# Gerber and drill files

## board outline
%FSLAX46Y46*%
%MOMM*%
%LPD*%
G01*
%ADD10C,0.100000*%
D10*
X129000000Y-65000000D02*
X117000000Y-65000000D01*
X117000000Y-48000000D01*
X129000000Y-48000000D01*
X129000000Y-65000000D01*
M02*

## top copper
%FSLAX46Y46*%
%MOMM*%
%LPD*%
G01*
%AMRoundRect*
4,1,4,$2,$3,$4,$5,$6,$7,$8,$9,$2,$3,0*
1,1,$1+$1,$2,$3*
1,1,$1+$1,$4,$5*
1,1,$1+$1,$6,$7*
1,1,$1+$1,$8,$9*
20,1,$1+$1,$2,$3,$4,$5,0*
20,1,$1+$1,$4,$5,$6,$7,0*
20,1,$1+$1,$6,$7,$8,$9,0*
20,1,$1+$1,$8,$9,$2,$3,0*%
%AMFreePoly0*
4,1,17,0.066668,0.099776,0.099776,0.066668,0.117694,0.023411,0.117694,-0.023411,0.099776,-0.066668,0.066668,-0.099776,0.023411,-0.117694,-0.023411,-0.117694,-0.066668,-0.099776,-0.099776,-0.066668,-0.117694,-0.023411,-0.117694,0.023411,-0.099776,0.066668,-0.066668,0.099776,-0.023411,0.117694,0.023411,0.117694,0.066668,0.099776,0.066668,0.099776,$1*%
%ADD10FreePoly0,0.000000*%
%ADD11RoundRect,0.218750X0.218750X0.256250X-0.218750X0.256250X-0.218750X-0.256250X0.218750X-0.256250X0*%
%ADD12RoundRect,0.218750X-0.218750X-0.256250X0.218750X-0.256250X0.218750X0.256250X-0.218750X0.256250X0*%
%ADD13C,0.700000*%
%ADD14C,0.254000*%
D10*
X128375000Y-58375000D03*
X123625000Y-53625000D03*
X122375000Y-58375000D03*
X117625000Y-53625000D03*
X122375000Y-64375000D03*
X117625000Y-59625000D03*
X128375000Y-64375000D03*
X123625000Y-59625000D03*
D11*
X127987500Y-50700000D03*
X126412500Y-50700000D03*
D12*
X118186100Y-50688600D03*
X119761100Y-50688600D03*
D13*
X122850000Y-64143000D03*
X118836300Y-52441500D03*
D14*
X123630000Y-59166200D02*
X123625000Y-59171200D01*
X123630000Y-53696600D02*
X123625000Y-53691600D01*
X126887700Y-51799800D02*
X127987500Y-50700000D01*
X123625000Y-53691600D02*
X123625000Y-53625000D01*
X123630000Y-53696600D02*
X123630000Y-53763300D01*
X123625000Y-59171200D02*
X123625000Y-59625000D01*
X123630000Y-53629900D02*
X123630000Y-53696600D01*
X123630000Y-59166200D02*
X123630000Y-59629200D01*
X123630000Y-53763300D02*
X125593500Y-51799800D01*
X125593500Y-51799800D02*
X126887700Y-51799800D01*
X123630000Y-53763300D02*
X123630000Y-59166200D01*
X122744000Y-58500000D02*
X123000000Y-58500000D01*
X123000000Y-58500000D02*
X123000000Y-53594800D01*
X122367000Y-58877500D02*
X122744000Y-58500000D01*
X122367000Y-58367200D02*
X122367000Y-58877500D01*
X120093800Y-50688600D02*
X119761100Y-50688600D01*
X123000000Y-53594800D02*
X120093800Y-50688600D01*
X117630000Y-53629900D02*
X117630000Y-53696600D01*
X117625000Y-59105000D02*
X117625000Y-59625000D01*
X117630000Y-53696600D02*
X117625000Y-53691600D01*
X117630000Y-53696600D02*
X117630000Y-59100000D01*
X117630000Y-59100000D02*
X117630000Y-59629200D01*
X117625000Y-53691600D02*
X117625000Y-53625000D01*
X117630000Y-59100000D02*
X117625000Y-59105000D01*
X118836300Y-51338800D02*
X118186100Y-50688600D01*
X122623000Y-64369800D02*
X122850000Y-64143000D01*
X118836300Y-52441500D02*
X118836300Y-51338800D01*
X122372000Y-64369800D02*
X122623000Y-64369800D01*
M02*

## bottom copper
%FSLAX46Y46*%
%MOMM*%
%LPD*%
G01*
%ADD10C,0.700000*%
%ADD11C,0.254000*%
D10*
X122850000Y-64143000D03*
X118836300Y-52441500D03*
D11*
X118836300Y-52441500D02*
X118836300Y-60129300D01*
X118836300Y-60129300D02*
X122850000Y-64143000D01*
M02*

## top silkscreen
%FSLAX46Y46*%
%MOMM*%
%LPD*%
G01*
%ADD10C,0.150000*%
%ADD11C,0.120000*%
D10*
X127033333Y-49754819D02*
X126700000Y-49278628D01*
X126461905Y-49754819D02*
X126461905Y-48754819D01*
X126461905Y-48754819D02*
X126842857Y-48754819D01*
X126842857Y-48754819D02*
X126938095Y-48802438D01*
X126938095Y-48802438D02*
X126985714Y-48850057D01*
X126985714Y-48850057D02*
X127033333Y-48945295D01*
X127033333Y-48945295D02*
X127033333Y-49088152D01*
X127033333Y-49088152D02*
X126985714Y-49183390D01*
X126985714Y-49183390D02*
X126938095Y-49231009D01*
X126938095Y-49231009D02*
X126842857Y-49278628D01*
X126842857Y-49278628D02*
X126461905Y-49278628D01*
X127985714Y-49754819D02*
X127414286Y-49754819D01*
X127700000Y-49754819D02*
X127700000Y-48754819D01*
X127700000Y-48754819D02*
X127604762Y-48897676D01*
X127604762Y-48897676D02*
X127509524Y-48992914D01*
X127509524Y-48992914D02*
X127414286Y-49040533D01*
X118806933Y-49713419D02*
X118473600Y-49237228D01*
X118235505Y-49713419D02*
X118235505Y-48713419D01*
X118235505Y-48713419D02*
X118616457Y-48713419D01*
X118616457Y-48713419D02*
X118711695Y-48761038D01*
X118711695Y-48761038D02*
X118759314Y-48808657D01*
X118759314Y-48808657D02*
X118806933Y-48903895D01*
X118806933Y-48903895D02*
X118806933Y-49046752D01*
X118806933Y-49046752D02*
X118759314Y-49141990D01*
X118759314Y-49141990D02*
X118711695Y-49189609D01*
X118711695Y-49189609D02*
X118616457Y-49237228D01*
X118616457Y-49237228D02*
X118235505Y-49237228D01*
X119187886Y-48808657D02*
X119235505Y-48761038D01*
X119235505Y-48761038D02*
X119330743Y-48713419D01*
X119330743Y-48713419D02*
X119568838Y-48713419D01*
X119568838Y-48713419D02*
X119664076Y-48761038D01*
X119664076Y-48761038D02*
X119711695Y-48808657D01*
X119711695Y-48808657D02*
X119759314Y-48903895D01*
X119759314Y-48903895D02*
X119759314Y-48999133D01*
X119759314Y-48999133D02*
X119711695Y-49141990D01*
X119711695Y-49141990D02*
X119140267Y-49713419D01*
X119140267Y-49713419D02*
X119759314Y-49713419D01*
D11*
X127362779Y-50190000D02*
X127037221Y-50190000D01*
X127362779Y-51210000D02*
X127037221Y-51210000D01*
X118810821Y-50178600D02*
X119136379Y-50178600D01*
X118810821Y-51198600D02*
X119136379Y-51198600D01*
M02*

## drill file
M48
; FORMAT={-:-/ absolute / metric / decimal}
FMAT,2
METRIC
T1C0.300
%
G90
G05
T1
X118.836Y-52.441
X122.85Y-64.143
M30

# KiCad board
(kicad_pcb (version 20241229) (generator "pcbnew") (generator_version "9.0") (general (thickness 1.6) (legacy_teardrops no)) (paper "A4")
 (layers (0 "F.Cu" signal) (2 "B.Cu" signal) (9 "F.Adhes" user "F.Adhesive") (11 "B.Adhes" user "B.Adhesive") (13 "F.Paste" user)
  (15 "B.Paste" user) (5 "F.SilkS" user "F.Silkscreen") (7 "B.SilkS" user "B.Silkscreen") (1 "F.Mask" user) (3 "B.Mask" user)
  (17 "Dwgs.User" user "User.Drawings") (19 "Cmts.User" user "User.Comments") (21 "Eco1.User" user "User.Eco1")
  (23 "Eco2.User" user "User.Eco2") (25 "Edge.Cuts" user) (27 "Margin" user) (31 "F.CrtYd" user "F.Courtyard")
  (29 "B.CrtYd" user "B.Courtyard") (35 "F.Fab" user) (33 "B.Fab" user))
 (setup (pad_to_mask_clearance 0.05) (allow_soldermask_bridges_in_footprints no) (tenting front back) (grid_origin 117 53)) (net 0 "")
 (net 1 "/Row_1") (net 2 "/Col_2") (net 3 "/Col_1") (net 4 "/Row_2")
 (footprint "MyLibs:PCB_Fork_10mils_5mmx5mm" (layer "F.Cu") (at 123.5 53.5)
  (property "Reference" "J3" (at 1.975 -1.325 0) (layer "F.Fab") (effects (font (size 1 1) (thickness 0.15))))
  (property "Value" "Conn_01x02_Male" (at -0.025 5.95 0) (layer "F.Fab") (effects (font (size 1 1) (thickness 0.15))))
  (pad "1" smd custom (at 4.875 4.875) (size 0.24 0.24) (layers "F.Cu" "F.Mask") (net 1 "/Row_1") (zone_connect 0) (thermal_bridge_angle 90)
   (options (clearance outline) (anchor circle)) (primitives))
  (pad "2" smd custom (at 0.125 0.125) (size 0.24 0.24) (layers "F.Cu" "F.Mask") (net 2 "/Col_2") (zone_connect 0) (thermal_bridge_angle 90)
   (options (clearance outline) (anchor circle)) (primitives)))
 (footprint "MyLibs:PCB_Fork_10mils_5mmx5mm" (layer "F.Cu") (at 117.5 53.5)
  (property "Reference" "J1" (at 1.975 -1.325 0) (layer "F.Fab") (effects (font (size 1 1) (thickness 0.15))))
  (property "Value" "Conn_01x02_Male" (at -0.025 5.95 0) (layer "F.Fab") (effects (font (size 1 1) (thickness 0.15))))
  (pad "1" smd custom (at 4.875 4.875) (size 0.24 0.24) (layers "F.Cu" "F.Mask") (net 1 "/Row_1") (zone_connect 0) (thermal_bridge_angle 90)
   (options (clearance outline) (anchor circle)) (primitives))
  (pad "2" smd custom (at 0.125 0.125) (size 0.24 0.24) (layers "F.Cu" "F.Mask") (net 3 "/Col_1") (zone_connect 0) (thermal_bridge_angle 90)
   (options (clearance outline) (anchor circle)) (primitives)))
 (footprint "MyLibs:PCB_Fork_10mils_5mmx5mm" (layer "F.Cu") (at 117.5 59.5)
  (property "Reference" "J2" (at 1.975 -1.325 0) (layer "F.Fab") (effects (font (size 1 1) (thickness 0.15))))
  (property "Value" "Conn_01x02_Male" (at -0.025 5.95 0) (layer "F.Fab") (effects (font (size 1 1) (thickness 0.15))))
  (pad "1" smd custom (at 4.875 4.875) (size 0.24 0.24) (layers "F.Cu" "F.Mask") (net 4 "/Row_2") (zone_connect 0) (thermal_bridge_angle 90)
   (options (clearance outline) (anchor circle)) (primitives))
  (pad "2" smd custom (at 0.125 0.125) (size 0.24 0.24) (layers "F.Cu" "F.Mask") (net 3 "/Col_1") (zone_connect 0) (thermal_bridge_angle 90)
   (options (clearance outline) (anchor circle)) (primitives)))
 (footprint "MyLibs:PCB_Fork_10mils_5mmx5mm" (layer "F.Cu") (at 123.5 59.5)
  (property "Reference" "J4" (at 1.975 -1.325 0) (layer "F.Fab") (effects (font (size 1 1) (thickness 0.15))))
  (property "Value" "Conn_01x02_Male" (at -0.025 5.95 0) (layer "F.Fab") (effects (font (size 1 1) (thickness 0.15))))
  (pad "1" smd custom (at 4.875 4.875) (size 0.24 0.24) (layers "F.Cu" "F.Mask") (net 4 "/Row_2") (zone_connect 0) (thermal_bridge_angle 90)
   (options (clearance outline) (anchor circle)) (primitives))
  (pad "2" smd custom (at 0.125 0.125) (size 0.24 0.24) (layers "F.Cu" "F.Mask") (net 2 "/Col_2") (zone_connect 0) (thermal_bridge_angle 90)
   (options (clearance outline) (anchor circle)) (primitives)))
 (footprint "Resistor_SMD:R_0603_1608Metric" (layer "F.Cu") (at 127.2 50.7 180)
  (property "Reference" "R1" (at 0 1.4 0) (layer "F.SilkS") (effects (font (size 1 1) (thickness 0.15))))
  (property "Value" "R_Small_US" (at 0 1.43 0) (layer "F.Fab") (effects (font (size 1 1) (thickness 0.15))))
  (fp_line (start -0.162779 0.51) (end 0.162779 0.51) (stroke (width 0.12) (type solid)) (layer "F.SilkS"))
  (fp_line (start -0.162779 -0.51) (end 0.162779 -0.51) (stroke (width 0.12) (type solid)) (layer "F.SilkS"))
  (pad "1" smd roundrect (at -0.7875 0 180) (size 0.875 0.95) (layers "F.Cu" "F.Mask" "F.Paste") (roundrect_rratio 0.25) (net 2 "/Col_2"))
  (pad "2" smd roundrect (at 0.7875 0 180) (size 0.875 0.95) (layers "F.Cu" "F.Mask" "F.Paste") (roundrect_rratio 0.25) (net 3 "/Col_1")))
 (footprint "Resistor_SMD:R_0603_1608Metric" (layer "F.Cu") (at 118.9736 50.6886)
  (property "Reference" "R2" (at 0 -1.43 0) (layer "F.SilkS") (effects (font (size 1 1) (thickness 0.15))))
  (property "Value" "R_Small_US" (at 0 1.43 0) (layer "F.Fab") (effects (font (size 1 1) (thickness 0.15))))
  (fp_line (start -0.162779 -0.51) (end 0.162779 -0.51) (stroke (width 0.12) (type solid)) (layer "F.SilkS"))
  (fp_line (start -0.162779 0.51) (end 0.162779 0.51) (stroke (width 0.12) (type solid)) (layer "F.SilkS"))
  (pad "1" smd roundrect (at -0.7875 0) (size 0.875 0.95) (layers "F.Cu" "F.Mask" "F.Paste") (roundrect_rratio 0.25) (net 4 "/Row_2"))
  (pad "2" smd roundrect (at 0.7875 0) (size 0.875 0.95) (layers "F.Cu" "F.Mask" "F.Paste") (roundrect_rratio 0.25) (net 1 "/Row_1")))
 (gr_poly (pts (xy 129 65) (xy 117 65) (xy 117 48) (xy 129 48)) (stroke (width 0.1) (type solid)) (fill no) (layer "Edge.Cuts"))
 (segment (start 123.63 59.1662) (end 123.625 59.1712) (width 0.254) (layer "F.Cu") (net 2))
 (segment (start 123.63 53.6966) (end 123.625 53.6916) (width 0.254) (layer "F.Cu") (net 2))
 (segment (start 126.8877 51.7998) (end 127.9875 50.7) (width 0.254) (layer "F.Cu") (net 2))
 (segment (start 123.625 53.6916) (end 123.625 53.625) (width 0.254) (layer "F.Cu") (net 2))
 (segment (start 123.63 53.6966) (end 123.63 53.7633) (width 0.254) (layer "F.Cu") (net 2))
 (segment (start 123.625 59.1712) (end 123.625 59.625) (width 0.254) (layer "F.Cu") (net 2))
 (segment (start 123.63 53.6299) (end 123.63 53.6966) (width 0.254) (layer "F.Cu") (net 2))
 (segment (start 123.63 59.1662) (end 123.63 59.6292) (width 0.254) (layer "F.Cu") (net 2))
 (segment (start 123.63 53.7633) (end 125.5935 51.7998) (width 0.254) (layer "F.Cu") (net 2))
 (segment (start 125.5935 51.7998) (end 126.8877 51.7998) (width 0.254) (layer "F.Cu") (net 2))
 (segment (start 123.63 53.7633) (end 123.63 59.1662) (width 0.254) (layer "F.Cu") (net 2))
 (segment (start 122.744 58.5) (end 123 58.5) (width 0.254) (layer "F.Cu") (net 1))
 (segment (start 123 58.5) (end 123 53.5948) (width 0.254) (layer "F.Cu") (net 1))
 (segment (start 122.367 58.8775) (end 122.744 58.5) (width 0.254) (layer "F.Cu") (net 1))
 (segment (start 122.367 58.3672) (end 122.367 58.8775) (width 0.254) (layer "F.Cu") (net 1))
 (segment (start 120.0938 50.6886) (end 119.7611 50.6886) (width 0.254) (layer "F.Cu") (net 1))
 (segment (start 123 53.5948) (end 120.0938 50.6886) (width 0.254) (layer "F.Cu") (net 1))
 (segment (start 117.63 53.6299) (end 117.63 53.6966) (width 0.254) (layer "F.Cu") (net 3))
 (segment (start 117.625 59.105) (end 117.625 59.625) (width 0.254) (layer "F.Cu") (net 3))
 (segment (start 117.63 53.6966) (end 117.625 53.6916) (width 0.254) (layer "F.Cu") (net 3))
 (segment (start 117.63 53.6966) (end 117.63 59.1) (width 0.254) (layer "F.Cu") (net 3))
 (segment (start 117.63 59.1) (end 117.63 59.6292) (width 0.254) (layer "F.Cu") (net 3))
 (segment (start 117.625 53.6916) (end 117.625 53.625) (width 0.254) (layer "F.Cu") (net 3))
 (segment (start 117.63 59.1) (end 117.625 59.105) (width 0.254) (layer "F.Cu") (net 3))
 (segment (start 118.8363 51.3388) (end 118.1861 50.6886) (width 0.254) (layer "F.Cu") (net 4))
 (segment (start 122.623 64.3698) (end 122.85 64.143) (width 0.254) (layer "F.Cu") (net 4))
 (segment (start 118.8363 52.4415) (end 118.8363 51.3388) (width 0.254) (layer "F.Cu") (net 4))
 (segment (start 122.372 64.3698) (end 122.623 64.3698) (width 0.254) (layer "F.Cu") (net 4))
 (via (at 122.85 64.143) (size 0.7) (drill 0.3) (layers "F.Cu" "B.Cu") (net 4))
 (via (at 118.8363 52.4415) (size 0.7) (drill 0.3) (layers "F.Cu" "B.Cu") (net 4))
 (segment (start 118.8363 52.4415) (end 118.8363 60.1293) (width 0.254) (layer "B.Cu") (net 4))
 (segment (start 118.8363 60.1293) (end 122.85 64.143) (width 0.254) (layer "B.Cu") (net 4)))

